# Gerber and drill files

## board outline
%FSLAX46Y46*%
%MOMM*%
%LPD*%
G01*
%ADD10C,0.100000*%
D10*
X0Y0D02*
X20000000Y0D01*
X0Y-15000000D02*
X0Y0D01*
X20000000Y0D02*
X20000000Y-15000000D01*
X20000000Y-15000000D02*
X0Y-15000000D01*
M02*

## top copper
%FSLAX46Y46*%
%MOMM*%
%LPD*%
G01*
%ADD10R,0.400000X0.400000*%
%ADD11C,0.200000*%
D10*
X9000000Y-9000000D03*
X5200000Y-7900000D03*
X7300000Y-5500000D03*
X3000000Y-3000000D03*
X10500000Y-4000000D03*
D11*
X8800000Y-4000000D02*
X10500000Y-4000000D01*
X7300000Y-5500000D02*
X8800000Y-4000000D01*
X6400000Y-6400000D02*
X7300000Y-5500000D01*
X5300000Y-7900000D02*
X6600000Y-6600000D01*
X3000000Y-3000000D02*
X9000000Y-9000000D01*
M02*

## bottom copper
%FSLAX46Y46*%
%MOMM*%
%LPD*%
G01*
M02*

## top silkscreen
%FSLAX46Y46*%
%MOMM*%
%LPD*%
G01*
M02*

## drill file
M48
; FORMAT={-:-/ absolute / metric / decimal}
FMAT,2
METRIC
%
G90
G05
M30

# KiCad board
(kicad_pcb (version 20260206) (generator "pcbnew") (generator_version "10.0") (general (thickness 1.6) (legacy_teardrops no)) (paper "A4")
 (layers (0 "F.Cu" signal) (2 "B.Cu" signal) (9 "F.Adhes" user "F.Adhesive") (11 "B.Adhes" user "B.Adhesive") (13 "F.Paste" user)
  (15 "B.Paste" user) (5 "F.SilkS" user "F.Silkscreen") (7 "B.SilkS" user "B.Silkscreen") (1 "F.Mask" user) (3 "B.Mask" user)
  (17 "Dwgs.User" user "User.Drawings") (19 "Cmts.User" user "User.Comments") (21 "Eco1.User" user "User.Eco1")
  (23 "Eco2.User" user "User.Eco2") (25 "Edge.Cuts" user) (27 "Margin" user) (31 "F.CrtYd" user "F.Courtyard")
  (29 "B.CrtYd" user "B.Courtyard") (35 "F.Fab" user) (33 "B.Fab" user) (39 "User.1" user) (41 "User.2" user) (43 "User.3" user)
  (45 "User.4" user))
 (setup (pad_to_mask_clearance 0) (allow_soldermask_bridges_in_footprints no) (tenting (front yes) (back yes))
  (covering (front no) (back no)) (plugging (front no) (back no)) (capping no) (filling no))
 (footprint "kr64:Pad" (layer "F.Cu") (at 9 9)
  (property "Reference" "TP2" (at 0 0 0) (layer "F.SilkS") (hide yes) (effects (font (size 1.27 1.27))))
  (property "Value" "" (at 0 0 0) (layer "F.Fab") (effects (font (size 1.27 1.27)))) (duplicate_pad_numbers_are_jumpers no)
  (pad "1" smd rect (at 0 0) (size 0.4 0.4) (layers "F.Cu" "F.Mask" "F.Paste") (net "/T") (thermal_bridge_angle 45)))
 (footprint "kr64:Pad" (layer "F.Cu") (at 5.2 7.9)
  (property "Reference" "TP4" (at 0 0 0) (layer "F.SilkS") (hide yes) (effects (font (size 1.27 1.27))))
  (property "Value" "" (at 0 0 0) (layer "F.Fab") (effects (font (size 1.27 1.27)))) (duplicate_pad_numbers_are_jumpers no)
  (pad "1" smd rect (at 0 0) (size 0.4 0.4) (layers "F.Cu" "F.Mask" "F.Paste") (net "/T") (thermal_bridge_angle 45)))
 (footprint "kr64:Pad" (layer "F.Cu") (at 7.3 5.5)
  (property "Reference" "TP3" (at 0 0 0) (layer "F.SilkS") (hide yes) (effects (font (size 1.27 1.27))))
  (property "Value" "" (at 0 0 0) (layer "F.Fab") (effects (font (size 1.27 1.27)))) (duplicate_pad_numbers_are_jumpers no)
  (pad "1" smd rect (at 0 0) (size 0.4 0.4) (layers "F.Cu" "F.Mask" "F.Paste") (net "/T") (thermal_bridge_angle 45)))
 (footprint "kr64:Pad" (layer "F.Cu") (at 3 3)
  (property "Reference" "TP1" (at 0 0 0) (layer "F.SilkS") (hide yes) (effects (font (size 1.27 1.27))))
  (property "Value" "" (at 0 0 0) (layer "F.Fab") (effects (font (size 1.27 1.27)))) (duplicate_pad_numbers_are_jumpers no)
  (pad "1" smd rect (at 0 0) (size 0.4 0.4) (layers "F.Cu" "F.Mask" "F.Paste") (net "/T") (thermal_bridge_angle 45)))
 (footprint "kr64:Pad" (layer "F.Cu") (at 10.5 4)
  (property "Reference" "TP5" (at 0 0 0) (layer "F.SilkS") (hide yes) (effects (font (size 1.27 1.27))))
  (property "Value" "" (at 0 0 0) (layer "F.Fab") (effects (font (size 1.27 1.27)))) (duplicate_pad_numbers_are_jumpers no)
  (pad "1" smd rect (at 0 0) (size 0.4 0.4) (layers "F.Cu" "F.Mask" "F.Paste") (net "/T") (thermal_bridge_angle 45)))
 (gr_line (start 0 0) (end 20 0) (stroke (width 0.1) (type default)) (layer "Edge.Cuts"))
 (gr_line (start 0 15) (end 0 0) (stroke (width 0.1) (type default)) (layer "Edge.Cuts"))
 (gr_line (start 20 0) (end 20 15) (stroke (width 0.1) (type default)) (layer "Edge.Cuts"))
 (gr_line (start 20 15) (end 0 15) (stroke (width 0.1) (type default)) (layer "Edge.Cuts"))
 (segment (start 8.8 4) (end 10.5 4) (width 0.2) (layer "F.Cu") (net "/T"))
 (segment (start 7.3 5.5) (end 8.8 4) (width 0.2) (layer "F.Cu") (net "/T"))
 (segment (start 6.4 6.4) (end 7.3 5.5) (width 0.2) (layer "F.Cu") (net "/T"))
 (segment (start 5.3 7.9) (end 6.6 6.6) (width 0.2) (layer "F.Cu") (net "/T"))
 (segment (start 3 3) (end 9 9) (width 0.2) (layer "F.Cu") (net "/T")))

